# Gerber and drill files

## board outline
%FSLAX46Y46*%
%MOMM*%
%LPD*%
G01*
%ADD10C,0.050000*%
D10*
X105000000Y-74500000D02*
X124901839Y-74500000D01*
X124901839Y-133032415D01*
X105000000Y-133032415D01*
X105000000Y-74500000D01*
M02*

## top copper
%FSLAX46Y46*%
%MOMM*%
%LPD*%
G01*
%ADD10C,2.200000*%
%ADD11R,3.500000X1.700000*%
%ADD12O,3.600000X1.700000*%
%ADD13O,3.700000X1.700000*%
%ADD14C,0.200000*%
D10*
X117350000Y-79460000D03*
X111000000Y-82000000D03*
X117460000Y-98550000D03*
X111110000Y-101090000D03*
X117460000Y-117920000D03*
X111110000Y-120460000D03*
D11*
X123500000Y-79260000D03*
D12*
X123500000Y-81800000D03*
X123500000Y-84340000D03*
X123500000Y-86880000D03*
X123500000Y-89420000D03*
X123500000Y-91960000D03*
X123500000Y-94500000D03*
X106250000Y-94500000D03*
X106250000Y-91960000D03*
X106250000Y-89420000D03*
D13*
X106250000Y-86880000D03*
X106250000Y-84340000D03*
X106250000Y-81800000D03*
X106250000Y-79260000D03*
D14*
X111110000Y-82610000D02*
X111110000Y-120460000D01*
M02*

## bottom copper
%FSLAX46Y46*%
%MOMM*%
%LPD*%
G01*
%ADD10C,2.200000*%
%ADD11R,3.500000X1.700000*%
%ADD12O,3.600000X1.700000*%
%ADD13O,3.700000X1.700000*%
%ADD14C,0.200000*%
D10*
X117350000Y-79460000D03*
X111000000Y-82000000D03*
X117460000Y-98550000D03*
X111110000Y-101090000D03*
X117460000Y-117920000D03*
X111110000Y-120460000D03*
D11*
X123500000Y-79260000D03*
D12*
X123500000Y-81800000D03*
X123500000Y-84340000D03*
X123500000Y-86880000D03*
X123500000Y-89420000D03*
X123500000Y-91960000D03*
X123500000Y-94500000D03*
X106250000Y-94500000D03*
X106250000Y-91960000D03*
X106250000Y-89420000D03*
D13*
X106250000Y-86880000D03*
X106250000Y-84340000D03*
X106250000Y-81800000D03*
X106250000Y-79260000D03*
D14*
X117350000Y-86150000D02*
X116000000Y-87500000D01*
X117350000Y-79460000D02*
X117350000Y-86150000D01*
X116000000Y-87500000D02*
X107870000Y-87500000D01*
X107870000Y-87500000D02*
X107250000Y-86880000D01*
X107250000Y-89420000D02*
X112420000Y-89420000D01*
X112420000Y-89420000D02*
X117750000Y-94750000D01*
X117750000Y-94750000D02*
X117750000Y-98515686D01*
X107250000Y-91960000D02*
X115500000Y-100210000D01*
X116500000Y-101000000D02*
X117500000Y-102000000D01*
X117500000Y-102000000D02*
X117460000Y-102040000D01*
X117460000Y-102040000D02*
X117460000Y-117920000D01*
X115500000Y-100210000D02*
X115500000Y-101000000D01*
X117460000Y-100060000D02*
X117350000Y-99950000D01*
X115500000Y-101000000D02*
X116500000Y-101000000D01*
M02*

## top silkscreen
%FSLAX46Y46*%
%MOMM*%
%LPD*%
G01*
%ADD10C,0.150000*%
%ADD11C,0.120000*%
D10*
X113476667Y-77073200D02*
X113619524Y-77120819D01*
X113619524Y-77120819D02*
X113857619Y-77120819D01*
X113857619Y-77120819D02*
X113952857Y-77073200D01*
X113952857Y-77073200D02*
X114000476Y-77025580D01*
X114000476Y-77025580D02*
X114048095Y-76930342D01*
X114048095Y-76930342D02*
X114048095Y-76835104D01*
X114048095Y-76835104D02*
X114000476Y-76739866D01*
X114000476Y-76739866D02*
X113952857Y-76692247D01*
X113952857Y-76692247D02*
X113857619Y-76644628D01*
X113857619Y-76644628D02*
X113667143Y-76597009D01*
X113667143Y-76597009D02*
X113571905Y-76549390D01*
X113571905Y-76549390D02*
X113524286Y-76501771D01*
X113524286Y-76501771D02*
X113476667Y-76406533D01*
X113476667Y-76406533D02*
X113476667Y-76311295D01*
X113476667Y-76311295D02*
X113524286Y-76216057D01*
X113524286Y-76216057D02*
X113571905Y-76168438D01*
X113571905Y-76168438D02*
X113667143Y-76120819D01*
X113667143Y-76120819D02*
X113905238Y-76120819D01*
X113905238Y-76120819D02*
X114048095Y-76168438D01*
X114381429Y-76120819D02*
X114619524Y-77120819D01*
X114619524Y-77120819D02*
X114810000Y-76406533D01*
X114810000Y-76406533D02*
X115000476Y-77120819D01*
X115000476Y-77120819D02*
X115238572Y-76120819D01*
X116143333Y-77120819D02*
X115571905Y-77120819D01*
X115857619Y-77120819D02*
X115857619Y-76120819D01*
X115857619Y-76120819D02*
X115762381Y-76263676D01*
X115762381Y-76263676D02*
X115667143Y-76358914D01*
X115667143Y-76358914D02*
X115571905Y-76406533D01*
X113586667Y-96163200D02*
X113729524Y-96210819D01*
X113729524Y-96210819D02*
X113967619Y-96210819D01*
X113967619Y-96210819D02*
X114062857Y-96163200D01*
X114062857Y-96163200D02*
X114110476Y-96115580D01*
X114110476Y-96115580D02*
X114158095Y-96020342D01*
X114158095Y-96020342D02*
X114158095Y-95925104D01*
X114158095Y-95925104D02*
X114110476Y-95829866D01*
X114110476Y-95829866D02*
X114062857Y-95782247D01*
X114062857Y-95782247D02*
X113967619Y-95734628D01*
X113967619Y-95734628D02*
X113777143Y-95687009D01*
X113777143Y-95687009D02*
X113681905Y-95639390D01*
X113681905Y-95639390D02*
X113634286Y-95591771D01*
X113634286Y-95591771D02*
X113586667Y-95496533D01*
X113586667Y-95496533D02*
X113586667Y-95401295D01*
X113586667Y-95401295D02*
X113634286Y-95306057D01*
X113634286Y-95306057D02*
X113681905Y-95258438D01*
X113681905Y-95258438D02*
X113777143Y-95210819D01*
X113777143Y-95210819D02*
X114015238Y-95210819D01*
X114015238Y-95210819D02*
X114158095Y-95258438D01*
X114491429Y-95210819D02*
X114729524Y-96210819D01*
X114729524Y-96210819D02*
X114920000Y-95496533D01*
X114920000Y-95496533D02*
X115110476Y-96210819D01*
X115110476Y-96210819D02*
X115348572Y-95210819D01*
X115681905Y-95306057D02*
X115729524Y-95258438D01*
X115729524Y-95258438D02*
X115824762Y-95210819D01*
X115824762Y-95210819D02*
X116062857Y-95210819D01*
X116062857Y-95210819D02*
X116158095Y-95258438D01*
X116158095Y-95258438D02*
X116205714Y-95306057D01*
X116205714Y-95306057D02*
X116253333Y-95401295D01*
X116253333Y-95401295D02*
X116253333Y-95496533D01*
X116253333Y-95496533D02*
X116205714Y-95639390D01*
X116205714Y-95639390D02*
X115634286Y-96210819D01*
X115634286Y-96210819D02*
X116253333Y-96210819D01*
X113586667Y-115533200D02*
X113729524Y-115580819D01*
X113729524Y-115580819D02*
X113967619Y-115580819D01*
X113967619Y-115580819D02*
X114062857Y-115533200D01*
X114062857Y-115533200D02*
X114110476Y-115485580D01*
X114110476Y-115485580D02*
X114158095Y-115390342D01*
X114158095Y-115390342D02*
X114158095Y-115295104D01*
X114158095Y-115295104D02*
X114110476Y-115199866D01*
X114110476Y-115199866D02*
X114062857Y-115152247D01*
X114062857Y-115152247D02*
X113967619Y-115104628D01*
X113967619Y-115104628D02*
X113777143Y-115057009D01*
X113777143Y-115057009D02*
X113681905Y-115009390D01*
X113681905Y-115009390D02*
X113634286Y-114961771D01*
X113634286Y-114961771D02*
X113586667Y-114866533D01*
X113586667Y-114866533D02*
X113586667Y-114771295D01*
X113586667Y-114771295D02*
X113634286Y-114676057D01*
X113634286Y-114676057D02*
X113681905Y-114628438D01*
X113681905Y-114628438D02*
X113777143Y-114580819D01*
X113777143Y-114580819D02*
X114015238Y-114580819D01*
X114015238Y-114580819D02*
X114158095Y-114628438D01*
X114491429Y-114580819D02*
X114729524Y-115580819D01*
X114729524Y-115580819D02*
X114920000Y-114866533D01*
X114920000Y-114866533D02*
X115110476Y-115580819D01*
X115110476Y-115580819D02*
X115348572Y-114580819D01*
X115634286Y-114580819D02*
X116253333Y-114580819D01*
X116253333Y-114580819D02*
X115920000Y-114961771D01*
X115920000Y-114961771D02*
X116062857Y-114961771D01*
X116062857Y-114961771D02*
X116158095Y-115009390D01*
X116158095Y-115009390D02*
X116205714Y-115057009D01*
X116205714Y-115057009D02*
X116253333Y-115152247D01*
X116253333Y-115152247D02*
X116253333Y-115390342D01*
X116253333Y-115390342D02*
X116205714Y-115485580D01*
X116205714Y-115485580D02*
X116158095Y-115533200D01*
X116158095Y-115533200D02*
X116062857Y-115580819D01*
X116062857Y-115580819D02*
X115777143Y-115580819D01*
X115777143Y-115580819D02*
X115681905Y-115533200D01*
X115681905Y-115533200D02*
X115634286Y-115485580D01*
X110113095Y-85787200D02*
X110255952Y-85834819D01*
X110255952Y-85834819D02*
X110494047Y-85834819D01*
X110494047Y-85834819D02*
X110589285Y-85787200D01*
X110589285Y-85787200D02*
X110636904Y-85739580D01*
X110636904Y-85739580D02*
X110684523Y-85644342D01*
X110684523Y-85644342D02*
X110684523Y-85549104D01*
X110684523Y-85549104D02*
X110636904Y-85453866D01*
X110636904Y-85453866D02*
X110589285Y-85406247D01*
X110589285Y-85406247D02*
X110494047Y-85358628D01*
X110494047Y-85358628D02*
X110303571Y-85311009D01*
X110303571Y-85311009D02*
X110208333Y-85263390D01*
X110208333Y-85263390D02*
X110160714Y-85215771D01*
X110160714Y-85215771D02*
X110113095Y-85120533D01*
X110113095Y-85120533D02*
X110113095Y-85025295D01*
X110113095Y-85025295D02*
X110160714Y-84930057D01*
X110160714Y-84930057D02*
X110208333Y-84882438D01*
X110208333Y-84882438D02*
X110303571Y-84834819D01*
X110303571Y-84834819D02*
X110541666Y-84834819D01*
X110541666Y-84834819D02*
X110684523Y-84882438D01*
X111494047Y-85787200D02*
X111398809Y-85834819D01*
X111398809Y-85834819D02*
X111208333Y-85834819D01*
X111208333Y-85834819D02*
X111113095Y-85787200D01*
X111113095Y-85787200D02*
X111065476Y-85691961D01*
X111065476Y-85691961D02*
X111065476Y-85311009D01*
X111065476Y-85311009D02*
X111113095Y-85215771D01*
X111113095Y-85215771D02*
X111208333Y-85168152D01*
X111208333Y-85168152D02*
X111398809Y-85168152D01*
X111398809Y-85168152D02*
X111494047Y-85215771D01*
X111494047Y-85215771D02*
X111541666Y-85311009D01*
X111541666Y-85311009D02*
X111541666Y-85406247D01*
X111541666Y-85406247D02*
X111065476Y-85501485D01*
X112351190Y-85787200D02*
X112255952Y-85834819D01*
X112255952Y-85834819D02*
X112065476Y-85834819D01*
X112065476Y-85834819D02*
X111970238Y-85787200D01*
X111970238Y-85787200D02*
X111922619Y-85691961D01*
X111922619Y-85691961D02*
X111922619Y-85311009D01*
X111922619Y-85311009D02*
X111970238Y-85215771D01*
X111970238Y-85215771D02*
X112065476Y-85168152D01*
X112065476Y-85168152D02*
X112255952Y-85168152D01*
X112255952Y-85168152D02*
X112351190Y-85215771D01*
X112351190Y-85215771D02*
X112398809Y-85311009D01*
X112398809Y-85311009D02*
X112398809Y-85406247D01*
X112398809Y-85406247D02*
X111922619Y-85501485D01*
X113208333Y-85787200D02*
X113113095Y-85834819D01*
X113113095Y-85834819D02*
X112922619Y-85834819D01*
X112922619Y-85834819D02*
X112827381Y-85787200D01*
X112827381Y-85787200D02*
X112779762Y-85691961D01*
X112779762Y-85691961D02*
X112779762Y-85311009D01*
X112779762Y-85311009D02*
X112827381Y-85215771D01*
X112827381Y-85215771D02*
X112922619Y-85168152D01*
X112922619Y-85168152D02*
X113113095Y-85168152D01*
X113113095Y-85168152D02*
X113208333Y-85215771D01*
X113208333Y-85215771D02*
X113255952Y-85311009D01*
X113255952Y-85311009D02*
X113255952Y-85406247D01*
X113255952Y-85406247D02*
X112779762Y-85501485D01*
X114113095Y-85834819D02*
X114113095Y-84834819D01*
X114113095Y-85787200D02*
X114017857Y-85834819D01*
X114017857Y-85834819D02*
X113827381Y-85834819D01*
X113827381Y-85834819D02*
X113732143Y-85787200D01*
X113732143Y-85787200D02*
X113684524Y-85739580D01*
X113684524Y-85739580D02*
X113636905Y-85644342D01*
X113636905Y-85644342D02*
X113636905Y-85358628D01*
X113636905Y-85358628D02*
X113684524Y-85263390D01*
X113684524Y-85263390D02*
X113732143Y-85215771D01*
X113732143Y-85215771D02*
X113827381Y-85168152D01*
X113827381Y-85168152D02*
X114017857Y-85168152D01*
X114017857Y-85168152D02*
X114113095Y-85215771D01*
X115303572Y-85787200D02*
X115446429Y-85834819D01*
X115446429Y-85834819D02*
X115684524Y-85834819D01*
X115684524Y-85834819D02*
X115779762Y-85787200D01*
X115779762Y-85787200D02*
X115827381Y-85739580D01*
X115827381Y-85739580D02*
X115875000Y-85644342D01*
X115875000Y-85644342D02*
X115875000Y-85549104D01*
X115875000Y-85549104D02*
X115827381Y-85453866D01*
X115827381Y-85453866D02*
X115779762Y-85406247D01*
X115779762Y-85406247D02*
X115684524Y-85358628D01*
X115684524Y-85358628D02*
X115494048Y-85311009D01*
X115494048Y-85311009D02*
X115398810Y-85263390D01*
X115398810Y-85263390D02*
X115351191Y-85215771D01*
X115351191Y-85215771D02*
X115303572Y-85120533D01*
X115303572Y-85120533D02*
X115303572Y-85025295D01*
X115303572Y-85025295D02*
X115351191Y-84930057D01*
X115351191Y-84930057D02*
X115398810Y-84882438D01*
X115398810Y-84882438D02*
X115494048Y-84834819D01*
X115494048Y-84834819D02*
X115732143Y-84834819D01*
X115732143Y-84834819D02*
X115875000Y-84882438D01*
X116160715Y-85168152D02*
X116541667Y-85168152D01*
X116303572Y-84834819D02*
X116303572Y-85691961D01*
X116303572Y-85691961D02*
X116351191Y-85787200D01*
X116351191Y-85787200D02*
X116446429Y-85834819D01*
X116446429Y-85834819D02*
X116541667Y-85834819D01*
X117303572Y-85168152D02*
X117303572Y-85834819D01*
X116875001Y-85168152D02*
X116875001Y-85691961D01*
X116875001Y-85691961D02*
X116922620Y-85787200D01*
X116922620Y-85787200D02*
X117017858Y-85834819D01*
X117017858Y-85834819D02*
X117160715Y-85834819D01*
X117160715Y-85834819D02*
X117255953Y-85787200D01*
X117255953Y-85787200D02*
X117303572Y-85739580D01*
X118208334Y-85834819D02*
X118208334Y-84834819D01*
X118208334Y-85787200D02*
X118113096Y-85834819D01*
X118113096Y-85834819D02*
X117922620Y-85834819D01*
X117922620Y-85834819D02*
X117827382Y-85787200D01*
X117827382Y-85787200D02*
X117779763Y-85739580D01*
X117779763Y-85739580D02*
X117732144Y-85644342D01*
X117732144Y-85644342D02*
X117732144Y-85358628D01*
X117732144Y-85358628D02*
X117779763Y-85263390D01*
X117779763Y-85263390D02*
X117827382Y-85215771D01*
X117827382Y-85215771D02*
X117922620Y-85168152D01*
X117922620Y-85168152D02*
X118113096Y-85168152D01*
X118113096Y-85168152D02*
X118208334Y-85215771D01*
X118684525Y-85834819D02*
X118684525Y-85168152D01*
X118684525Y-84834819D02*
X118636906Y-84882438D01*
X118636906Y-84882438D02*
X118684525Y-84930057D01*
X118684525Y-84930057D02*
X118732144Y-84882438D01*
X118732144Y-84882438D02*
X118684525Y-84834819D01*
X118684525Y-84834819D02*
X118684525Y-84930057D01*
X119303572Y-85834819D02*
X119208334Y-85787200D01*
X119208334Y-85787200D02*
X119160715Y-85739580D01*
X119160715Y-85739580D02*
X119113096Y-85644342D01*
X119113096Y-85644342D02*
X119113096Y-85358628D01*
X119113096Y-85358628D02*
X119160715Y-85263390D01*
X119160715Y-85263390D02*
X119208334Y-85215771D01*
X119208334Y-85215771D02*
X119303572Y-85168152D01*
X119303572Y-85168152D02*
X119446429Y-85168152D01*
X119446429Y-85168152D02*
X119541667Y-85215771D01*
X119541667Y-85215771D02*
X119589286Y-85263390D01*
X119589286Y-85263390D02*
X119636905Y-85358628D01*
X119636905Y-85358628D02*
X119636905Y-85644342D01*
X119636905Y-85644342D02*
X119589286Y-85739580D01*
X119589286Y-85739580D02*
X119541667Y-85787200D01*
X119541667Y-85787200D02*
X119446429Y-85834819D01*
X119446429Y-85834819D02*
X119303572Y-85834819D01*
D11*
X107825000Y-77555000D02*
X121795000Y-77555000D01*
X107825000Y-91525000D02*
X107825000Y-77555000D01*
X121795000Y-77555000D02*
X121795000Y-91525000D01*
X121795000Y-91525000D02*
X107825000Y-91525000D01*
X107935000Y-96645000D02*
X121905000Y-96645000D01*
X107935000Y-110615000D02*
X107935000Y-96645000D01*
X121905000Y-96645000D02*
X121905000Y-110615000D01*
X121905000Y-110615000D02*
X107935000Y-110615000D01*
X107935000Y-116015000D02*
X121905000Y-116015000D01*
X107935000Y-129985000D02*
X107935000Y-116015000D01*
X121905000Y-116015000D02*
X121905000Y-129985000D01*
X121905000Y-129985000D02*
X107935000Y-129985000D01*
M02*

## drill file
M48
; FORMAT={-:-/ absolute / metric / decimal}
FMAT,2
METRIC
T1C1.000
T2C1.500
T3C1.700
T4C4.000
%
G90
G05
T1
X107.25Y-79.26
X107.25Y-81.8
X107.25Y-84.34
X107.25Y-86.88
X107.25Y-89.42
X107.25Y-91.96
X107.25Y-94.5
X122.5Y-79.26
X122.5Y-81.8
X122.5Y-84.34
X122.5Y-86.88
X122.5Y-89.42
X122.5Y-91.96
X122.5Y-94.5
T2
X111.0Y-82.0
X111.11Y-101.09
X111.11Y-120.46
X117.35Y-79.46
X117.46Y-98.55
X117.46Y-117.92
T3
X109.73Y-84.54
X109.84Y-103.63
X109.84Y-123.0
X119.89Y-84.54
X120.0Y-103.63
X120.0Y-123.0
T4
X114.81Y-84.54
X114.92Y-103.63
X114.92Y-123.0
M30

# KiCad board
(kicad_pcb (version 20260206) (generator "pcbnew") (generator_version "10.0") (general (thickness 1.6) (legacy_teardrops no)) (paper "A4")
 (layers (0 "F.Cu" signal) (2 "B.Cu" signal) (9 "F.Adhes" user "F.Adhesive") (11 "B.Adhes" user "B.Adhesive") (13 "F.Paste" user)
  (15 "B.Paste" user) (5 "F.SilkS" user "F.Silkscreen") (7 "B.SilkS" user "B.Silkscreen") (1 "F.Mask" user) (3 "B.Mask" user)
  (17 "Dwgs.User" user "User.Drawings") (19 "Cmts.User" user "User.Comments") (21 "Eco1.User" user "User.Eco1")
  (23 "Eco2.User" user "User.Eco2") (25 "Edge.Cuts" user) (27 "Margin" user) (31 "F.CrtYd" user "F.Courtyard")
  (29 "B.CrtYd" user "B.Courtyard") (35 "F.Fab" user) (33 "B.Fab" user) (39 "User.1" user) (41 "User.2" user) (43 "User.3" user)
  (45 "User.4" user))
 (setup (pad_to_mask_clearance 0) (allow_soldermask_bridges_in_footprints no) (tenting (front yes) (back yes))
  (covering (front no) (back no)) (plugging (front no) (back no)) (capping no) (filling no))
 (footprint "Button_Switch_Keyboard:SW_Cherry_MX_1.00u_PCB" (layer "F.Cu") (at 117.35 79.46)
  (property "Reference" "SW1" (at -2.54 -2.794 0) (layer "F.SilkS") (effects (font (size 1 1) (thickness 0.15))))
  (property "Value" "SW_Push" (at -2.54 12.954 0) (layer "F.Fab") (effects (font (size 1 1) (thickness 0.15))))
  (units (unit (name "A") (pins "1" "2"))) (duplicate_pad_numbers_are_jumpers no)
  (fp_line (start -9.525 -1.905) (end 4.445 -1.905) (stroke (width 0.12) (type solid)) (layer "F.SilkS"))
  (fp_line (start -9.525 12.065) (end -9.525 -1.905) (stroke (width 0.12) (type solid)) (layer "F.SilkS"))
  (fp_line (start 4.445 -1.905) (end 4.445 12.065) (stroke (width 0.12) (type solid)) (layer "F.SilkS"))
  (fp_line (start 4.445 12.065) (end -9.525 12.065) (stroke (width 0.12) (type solid)) (layer "F.SilkS"))
  (pad "" np_thru_hole circle (at -7.62 5.08) (size 1.7 1.7) (drill 1.7) (layers "*.Cu" "*.Mask"))
  (pad "" np_thru_hole circle (at -2.54 5.08) (size 4 4) (drill 4) (layers "*.Cu" "*.Mask"))
  (pad "" np_thru_hole circle (at 2.54 5.08) (size 1.7 1.7) (drill 1.7) (layers "*.Cu" "*.Mask"))
  (pad "1" thru_hole circle (at 0 0) (size 2.2 2.2) (drill 1.5) (layers "*.Cu" "*.Mask") (remove_unused_layers no)
   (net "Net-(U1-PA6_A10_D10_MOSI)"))
  (pad "2" thru_hole circle (at -6.35 2.54) (size 2.2 2.2) (drill 1.5) (layers "*.Cu" "*.Mask") (remove_unused_layers no) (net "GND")))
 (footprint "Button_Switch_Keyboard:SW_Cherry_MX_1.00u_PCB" (layer "F.Cu") (at 117.46 98.55)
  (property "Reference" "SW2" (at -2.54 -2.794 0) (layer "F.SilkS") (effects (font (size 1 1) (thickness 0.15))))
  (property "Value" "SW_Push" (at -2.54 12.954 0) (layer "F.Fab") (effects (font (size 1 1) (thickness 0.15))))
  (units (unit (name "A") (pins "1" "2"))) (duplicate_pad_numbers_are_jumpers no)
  (fp_line (start -9.525 -1.905) (end 4.445 -1.905) (stroke (width 0.12) (type solid)) (layer "F.SilkS"))
  (fp_line (start -9.525 12.065) (end -9.525 -1.905) (stroke (width 0.12) (type solid)) (layer "F.SilkS"))
  (fp_line (start 4.445 -1.905) (end 4.445 12.065) (stroke (width 0.12) (type solid)) (layer "F.SilkS"))
  (fp_line (start 4.445 12.065) (end -9.525 12.065) (stroke (width 0.12) (type solid)) (layer "F.SilkS"))
  (pad "" np_thru_hole circle (at -7.62 5.08) (size 1.7 1.7) (drill 1.7) (layers "*.Cu" "*.Mask"))
  (pad "" np_thru_hole circle (at -2.54 5.08) (size 4 4) (drill 4) (layers "*.Cu" "*.Mask"))
  (pad "" np_thru_hole circle (at 2.54 5.08) (size 1.7 1.7) (drill 1.7) (layers "*.Cu" "*.Mask"))
  (pad "1" thru_hole circle (at 0 0) (size 2.2 2.2) (drill 1.5) (layers "*.Cu" "*.Mask") (remove_unused_layers no)
   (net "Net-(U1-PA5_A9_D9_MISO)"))
  (pad "2" thru_hole circle (at -6.35 2.54) (size 2.2 2.2) (drill 1.5) (layers "*.Cu" "*.Mask") (remove_unused_layers no) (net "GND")))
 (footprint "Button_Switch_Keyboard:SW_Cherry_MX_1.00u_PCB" (layer "F.Cu") (at 117.46 117.92)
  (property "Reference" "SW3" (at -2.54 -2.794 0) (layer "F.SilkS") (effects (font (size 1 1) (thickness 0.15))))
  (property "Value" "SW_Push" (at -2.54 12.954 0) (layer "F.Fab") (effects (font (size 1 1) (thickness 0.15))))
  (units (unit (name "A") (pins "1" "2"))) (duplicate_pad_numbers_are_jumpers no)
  (fp_line (start -9.525 -1.905) (end 4.445 -1.905) (stroke (width 0.12) (type solid)) (layer "F.SilkS"))
  (fp_line (start -9.525 12.065) (end -9.525 -1.905) (stroke (width 0.12) (type solid)) (layer "F.SilkS"))
  (fp_line (start 4.445 -1.905) (end 4.445 12.065) (stroke (width 0.12) (type solid)) (layer "F.SilkS"))
  (fp_line (start 4.445 12.065) (end -9.525 12.065) (stroke (width 0.12) (type solid)) (layer "F.SilkS"))
  (pad "" np_thru_hole circle (at -7.62 5.08) (size 1.7 1.7) (drill 1.7) (layers "*.Cu" "*.Mask"))
  (pad "" np_thru_hole circle (at -2.54 5.08) (size 4 4) (drill 4) (layers "*.Cu" "*.Mask"))
  (pad "" np_thru_hole circle (at 2.54 5.08) (size 1.7 1.7) (drill 1.7) (layers "*.Cu" "*.Mask"))
  (pad "1" thru_hole circle (at 0 0) (size 2.2 2.2) (drill 1.5) (layers "*.Cu" "*.Mask") (remove_unused_layers no)
   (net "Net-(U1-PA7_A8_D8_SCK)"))
  (pad "2" thru_hole circle (at -6.35 2.54) (size 2.2 2.2) (drill 1.5) (layers "*.Cu" "*.Mask") (remove_unused_layers no) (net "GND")))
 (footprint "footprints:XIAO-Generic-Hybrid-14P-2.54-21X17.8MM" (layer "B.Cu") (at 114.875 86.88 180)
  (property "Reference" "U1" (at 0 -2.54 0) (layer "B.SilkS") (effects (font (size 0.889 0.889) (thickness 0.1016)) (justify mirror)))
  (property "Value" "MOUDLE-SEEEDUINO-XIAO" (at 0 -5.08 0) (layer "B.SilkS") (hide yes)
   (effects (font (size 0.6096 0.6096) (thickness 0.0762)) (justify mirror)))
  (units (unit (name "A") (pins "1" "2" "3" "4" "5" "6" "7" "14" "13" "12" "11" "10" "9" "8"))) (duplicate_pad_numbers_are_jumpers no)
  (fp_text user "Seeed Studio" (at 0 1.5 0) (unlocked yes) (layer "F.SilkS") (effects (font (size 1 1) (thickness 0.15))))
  (pad "1" thru_hole rect (at -7.625 7.62 180) (size 3.5 1.7) (drill 1 (offset -1 0)) (layers "*.Cu" "*.Mask") (remove_unused_layers no)
   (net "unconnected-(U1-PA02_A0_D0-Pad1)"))
  (pad "2" thru_hole oval (at -7.625 5.08 180) (size 3.6 1.7) (drill 1 (offset -1 0)) (layers "*.Cu" "*.Mask") (remove_unused_layers no)
   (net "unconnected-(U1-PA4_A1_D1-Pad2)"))
  (pad "3" thru_hole oval (at -7.625 2.54 180) (size 3.6 1.7) (drill 1 (offset -1 0)) (layers "*.Cu" "*.Mask") (remove_unused_layers no)
   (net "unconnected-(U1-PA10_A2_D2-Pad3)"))
  (pad "4" thru_hole oval (at -7.625 0 180) (size 3.6 1.7) (drill 1 (offset -1 0)) (layers "*.Cu" "*.Mask") (remove_unused_layers no)
   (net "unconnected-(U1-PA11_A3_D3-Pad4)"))
  (pad "5" thru_hole oval (at -7.625 -2.54 180) (size 3.6 1.7) (drill 1 (offset -1 0)) (layers "*.Cu" "*.Mask") (remove_unused_layers no)
   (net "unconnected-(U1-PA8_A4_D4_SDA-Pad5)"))
  (pad "6" thru_hole oval (at -7.625 -5.08) (size 3.6 1.7) (drill 1 (offset 1 0)) (layers "*.Cu" "*.Mask") (remove_unused_layers no)
   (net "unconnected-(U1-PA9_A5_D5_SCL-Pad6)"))
  (pad "7" thru_hole oval (at -7.625 -7.62 180) (size 3.6 1.7) (drill 1 (offset -1 0)) (layers "*.Cu" "*.Mask") (remove_unused_layers no)
   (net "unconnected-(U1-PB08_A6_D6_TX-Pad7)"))
  (pad "8" thru_hole oval (at 7.625 -7.62 180) (size 3.6 1.7) (drill 1 (offset 1 0)) (layers "*.Cu" "*.Mask") (remove_unused_layers no)
   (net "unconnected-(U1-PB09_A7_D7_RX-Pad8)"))
  (pad "9" thru_hole oval (at 7.625 -5.08 180) (size 3.6 1.7) (drill 1 (offset 1 0)) (layers "*.Cu" "*.Mask") (remove_unused_layers no)
   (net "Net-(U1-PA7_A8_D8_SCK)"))
  (pad "10" thru_hole oval (at 7.625 -2.54 180) (size 3.6 1.7) (drill 1 (offset 1 0)) (layers "*.Cu" "*.Mask") (remove_unused_layers no)
   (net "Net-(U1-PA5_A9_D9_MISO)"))
  (pad "11" thru_hole oval (at 7.625 0 180) (size 3.7 1.7) (drill 1 (offset 1 0)) (layers "*.Cu" "*.Mask") (remove_unused_layers no)
   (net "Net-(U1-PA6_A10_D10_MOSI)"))
  (pad "12" thru_hole oval (at 7.625 2.54 180) (size 3.7 1.7) (drill 1 (offset 1 0)) (layers "*.Cu" "*.Mask") (remove_unused_layers no)
   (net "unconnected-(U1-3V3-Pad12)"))
  (pad "13" thru_hole oval (at 7.625 5.08 180) (size 3.7 1.7) (drill 1 (offset 1 0)) (layers "*.Cu" "*.Mask") (remove_unused_layers no)
   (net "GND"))
  (pad "14" thru_hole oval (at 7.625 7.62 180) (size 3.7 1.7) (drill 1 (offset 1 0)) (layers "*.Cu" "*.Mask") (remove_unused_layers no)
   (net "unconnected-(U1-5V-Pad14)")))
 (gr_rect (start 105 74.5) (end 124.901839 133.032415) (stroke (width 0.05) (type default)) (fill no) (layer "Edge.Cuts"))
 (segment (start 117.35 86.15) (end 116 87.5) (width 0.2) (layer "B.Cu") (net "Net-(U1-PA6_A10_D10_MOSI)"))
 (segment (start 117.35 79.46) (end 117.35 86.15) (width 0.2) (layer "B.Cu") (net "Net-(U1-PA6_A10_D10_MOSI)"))
 (segment (start 116 87.5) (end 107.87 87.5) (width 0.2) (layer "B.Cu") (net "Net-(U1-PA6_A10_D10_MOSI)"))
 (segment (start 107.87 87.5) (end 107.25 86.88) (width 0.2) (layer "B.Cu") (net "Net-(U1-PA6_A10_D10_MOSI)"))
 (segment (start 111.11 82.61) (end 111.11 120.46) (width 0.2) (layer "F.Cu") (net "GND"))
 (segment (start 107.25 89.42) (end 112.42 89.42) (width 0.2) (layer "B.Cu") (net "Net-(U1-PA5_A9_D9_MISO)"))
 (segment (start 112.42 89.42) (end 117.75 94.75) (width 0.2) (layer "B.Cu") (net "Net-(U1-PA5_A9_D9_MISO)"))
 (segment (start 117.75 94.75) (end 117.75 98.515686) (width 0.2) (layer "B.Cu") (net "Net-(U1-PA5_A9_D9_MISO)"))
 (segment (start 107.25 91.96) (end 115.5 100.21) (width 0.2) (layer "B.Cu") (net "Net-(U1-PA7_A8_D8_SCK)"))
 (segment (start 116.5 101) (end 117.5 102) (width 0.2) (layer "B.Cu") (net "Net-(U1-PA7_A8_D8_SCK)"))
 (segment (start 117.5 102) (end 117.46 102.04) (width 0.2) (layer "B.Cu") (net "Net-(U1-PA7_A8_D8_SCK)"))
 (segment (start 117.46 102.04) (end 117.46 117.92) (width 0.2) (layer "B.Cu") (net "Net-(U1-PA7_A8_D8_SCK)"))
 (segment (start 115.5 100.21) (end 115.5 101) (width 0.2) (layer "B.Cu") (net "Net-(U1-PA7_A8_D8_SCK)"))
 (segment (start 117.46 100.06) (end 117.35 99.95) (width 0.2) (layer "B.Cu") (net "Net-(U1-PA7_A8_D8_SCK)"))
 (segment (start 115.5 101) (end 116.5 101) (width 0.2) (layer "B.Cu") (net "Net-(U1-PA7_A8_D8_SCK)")))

